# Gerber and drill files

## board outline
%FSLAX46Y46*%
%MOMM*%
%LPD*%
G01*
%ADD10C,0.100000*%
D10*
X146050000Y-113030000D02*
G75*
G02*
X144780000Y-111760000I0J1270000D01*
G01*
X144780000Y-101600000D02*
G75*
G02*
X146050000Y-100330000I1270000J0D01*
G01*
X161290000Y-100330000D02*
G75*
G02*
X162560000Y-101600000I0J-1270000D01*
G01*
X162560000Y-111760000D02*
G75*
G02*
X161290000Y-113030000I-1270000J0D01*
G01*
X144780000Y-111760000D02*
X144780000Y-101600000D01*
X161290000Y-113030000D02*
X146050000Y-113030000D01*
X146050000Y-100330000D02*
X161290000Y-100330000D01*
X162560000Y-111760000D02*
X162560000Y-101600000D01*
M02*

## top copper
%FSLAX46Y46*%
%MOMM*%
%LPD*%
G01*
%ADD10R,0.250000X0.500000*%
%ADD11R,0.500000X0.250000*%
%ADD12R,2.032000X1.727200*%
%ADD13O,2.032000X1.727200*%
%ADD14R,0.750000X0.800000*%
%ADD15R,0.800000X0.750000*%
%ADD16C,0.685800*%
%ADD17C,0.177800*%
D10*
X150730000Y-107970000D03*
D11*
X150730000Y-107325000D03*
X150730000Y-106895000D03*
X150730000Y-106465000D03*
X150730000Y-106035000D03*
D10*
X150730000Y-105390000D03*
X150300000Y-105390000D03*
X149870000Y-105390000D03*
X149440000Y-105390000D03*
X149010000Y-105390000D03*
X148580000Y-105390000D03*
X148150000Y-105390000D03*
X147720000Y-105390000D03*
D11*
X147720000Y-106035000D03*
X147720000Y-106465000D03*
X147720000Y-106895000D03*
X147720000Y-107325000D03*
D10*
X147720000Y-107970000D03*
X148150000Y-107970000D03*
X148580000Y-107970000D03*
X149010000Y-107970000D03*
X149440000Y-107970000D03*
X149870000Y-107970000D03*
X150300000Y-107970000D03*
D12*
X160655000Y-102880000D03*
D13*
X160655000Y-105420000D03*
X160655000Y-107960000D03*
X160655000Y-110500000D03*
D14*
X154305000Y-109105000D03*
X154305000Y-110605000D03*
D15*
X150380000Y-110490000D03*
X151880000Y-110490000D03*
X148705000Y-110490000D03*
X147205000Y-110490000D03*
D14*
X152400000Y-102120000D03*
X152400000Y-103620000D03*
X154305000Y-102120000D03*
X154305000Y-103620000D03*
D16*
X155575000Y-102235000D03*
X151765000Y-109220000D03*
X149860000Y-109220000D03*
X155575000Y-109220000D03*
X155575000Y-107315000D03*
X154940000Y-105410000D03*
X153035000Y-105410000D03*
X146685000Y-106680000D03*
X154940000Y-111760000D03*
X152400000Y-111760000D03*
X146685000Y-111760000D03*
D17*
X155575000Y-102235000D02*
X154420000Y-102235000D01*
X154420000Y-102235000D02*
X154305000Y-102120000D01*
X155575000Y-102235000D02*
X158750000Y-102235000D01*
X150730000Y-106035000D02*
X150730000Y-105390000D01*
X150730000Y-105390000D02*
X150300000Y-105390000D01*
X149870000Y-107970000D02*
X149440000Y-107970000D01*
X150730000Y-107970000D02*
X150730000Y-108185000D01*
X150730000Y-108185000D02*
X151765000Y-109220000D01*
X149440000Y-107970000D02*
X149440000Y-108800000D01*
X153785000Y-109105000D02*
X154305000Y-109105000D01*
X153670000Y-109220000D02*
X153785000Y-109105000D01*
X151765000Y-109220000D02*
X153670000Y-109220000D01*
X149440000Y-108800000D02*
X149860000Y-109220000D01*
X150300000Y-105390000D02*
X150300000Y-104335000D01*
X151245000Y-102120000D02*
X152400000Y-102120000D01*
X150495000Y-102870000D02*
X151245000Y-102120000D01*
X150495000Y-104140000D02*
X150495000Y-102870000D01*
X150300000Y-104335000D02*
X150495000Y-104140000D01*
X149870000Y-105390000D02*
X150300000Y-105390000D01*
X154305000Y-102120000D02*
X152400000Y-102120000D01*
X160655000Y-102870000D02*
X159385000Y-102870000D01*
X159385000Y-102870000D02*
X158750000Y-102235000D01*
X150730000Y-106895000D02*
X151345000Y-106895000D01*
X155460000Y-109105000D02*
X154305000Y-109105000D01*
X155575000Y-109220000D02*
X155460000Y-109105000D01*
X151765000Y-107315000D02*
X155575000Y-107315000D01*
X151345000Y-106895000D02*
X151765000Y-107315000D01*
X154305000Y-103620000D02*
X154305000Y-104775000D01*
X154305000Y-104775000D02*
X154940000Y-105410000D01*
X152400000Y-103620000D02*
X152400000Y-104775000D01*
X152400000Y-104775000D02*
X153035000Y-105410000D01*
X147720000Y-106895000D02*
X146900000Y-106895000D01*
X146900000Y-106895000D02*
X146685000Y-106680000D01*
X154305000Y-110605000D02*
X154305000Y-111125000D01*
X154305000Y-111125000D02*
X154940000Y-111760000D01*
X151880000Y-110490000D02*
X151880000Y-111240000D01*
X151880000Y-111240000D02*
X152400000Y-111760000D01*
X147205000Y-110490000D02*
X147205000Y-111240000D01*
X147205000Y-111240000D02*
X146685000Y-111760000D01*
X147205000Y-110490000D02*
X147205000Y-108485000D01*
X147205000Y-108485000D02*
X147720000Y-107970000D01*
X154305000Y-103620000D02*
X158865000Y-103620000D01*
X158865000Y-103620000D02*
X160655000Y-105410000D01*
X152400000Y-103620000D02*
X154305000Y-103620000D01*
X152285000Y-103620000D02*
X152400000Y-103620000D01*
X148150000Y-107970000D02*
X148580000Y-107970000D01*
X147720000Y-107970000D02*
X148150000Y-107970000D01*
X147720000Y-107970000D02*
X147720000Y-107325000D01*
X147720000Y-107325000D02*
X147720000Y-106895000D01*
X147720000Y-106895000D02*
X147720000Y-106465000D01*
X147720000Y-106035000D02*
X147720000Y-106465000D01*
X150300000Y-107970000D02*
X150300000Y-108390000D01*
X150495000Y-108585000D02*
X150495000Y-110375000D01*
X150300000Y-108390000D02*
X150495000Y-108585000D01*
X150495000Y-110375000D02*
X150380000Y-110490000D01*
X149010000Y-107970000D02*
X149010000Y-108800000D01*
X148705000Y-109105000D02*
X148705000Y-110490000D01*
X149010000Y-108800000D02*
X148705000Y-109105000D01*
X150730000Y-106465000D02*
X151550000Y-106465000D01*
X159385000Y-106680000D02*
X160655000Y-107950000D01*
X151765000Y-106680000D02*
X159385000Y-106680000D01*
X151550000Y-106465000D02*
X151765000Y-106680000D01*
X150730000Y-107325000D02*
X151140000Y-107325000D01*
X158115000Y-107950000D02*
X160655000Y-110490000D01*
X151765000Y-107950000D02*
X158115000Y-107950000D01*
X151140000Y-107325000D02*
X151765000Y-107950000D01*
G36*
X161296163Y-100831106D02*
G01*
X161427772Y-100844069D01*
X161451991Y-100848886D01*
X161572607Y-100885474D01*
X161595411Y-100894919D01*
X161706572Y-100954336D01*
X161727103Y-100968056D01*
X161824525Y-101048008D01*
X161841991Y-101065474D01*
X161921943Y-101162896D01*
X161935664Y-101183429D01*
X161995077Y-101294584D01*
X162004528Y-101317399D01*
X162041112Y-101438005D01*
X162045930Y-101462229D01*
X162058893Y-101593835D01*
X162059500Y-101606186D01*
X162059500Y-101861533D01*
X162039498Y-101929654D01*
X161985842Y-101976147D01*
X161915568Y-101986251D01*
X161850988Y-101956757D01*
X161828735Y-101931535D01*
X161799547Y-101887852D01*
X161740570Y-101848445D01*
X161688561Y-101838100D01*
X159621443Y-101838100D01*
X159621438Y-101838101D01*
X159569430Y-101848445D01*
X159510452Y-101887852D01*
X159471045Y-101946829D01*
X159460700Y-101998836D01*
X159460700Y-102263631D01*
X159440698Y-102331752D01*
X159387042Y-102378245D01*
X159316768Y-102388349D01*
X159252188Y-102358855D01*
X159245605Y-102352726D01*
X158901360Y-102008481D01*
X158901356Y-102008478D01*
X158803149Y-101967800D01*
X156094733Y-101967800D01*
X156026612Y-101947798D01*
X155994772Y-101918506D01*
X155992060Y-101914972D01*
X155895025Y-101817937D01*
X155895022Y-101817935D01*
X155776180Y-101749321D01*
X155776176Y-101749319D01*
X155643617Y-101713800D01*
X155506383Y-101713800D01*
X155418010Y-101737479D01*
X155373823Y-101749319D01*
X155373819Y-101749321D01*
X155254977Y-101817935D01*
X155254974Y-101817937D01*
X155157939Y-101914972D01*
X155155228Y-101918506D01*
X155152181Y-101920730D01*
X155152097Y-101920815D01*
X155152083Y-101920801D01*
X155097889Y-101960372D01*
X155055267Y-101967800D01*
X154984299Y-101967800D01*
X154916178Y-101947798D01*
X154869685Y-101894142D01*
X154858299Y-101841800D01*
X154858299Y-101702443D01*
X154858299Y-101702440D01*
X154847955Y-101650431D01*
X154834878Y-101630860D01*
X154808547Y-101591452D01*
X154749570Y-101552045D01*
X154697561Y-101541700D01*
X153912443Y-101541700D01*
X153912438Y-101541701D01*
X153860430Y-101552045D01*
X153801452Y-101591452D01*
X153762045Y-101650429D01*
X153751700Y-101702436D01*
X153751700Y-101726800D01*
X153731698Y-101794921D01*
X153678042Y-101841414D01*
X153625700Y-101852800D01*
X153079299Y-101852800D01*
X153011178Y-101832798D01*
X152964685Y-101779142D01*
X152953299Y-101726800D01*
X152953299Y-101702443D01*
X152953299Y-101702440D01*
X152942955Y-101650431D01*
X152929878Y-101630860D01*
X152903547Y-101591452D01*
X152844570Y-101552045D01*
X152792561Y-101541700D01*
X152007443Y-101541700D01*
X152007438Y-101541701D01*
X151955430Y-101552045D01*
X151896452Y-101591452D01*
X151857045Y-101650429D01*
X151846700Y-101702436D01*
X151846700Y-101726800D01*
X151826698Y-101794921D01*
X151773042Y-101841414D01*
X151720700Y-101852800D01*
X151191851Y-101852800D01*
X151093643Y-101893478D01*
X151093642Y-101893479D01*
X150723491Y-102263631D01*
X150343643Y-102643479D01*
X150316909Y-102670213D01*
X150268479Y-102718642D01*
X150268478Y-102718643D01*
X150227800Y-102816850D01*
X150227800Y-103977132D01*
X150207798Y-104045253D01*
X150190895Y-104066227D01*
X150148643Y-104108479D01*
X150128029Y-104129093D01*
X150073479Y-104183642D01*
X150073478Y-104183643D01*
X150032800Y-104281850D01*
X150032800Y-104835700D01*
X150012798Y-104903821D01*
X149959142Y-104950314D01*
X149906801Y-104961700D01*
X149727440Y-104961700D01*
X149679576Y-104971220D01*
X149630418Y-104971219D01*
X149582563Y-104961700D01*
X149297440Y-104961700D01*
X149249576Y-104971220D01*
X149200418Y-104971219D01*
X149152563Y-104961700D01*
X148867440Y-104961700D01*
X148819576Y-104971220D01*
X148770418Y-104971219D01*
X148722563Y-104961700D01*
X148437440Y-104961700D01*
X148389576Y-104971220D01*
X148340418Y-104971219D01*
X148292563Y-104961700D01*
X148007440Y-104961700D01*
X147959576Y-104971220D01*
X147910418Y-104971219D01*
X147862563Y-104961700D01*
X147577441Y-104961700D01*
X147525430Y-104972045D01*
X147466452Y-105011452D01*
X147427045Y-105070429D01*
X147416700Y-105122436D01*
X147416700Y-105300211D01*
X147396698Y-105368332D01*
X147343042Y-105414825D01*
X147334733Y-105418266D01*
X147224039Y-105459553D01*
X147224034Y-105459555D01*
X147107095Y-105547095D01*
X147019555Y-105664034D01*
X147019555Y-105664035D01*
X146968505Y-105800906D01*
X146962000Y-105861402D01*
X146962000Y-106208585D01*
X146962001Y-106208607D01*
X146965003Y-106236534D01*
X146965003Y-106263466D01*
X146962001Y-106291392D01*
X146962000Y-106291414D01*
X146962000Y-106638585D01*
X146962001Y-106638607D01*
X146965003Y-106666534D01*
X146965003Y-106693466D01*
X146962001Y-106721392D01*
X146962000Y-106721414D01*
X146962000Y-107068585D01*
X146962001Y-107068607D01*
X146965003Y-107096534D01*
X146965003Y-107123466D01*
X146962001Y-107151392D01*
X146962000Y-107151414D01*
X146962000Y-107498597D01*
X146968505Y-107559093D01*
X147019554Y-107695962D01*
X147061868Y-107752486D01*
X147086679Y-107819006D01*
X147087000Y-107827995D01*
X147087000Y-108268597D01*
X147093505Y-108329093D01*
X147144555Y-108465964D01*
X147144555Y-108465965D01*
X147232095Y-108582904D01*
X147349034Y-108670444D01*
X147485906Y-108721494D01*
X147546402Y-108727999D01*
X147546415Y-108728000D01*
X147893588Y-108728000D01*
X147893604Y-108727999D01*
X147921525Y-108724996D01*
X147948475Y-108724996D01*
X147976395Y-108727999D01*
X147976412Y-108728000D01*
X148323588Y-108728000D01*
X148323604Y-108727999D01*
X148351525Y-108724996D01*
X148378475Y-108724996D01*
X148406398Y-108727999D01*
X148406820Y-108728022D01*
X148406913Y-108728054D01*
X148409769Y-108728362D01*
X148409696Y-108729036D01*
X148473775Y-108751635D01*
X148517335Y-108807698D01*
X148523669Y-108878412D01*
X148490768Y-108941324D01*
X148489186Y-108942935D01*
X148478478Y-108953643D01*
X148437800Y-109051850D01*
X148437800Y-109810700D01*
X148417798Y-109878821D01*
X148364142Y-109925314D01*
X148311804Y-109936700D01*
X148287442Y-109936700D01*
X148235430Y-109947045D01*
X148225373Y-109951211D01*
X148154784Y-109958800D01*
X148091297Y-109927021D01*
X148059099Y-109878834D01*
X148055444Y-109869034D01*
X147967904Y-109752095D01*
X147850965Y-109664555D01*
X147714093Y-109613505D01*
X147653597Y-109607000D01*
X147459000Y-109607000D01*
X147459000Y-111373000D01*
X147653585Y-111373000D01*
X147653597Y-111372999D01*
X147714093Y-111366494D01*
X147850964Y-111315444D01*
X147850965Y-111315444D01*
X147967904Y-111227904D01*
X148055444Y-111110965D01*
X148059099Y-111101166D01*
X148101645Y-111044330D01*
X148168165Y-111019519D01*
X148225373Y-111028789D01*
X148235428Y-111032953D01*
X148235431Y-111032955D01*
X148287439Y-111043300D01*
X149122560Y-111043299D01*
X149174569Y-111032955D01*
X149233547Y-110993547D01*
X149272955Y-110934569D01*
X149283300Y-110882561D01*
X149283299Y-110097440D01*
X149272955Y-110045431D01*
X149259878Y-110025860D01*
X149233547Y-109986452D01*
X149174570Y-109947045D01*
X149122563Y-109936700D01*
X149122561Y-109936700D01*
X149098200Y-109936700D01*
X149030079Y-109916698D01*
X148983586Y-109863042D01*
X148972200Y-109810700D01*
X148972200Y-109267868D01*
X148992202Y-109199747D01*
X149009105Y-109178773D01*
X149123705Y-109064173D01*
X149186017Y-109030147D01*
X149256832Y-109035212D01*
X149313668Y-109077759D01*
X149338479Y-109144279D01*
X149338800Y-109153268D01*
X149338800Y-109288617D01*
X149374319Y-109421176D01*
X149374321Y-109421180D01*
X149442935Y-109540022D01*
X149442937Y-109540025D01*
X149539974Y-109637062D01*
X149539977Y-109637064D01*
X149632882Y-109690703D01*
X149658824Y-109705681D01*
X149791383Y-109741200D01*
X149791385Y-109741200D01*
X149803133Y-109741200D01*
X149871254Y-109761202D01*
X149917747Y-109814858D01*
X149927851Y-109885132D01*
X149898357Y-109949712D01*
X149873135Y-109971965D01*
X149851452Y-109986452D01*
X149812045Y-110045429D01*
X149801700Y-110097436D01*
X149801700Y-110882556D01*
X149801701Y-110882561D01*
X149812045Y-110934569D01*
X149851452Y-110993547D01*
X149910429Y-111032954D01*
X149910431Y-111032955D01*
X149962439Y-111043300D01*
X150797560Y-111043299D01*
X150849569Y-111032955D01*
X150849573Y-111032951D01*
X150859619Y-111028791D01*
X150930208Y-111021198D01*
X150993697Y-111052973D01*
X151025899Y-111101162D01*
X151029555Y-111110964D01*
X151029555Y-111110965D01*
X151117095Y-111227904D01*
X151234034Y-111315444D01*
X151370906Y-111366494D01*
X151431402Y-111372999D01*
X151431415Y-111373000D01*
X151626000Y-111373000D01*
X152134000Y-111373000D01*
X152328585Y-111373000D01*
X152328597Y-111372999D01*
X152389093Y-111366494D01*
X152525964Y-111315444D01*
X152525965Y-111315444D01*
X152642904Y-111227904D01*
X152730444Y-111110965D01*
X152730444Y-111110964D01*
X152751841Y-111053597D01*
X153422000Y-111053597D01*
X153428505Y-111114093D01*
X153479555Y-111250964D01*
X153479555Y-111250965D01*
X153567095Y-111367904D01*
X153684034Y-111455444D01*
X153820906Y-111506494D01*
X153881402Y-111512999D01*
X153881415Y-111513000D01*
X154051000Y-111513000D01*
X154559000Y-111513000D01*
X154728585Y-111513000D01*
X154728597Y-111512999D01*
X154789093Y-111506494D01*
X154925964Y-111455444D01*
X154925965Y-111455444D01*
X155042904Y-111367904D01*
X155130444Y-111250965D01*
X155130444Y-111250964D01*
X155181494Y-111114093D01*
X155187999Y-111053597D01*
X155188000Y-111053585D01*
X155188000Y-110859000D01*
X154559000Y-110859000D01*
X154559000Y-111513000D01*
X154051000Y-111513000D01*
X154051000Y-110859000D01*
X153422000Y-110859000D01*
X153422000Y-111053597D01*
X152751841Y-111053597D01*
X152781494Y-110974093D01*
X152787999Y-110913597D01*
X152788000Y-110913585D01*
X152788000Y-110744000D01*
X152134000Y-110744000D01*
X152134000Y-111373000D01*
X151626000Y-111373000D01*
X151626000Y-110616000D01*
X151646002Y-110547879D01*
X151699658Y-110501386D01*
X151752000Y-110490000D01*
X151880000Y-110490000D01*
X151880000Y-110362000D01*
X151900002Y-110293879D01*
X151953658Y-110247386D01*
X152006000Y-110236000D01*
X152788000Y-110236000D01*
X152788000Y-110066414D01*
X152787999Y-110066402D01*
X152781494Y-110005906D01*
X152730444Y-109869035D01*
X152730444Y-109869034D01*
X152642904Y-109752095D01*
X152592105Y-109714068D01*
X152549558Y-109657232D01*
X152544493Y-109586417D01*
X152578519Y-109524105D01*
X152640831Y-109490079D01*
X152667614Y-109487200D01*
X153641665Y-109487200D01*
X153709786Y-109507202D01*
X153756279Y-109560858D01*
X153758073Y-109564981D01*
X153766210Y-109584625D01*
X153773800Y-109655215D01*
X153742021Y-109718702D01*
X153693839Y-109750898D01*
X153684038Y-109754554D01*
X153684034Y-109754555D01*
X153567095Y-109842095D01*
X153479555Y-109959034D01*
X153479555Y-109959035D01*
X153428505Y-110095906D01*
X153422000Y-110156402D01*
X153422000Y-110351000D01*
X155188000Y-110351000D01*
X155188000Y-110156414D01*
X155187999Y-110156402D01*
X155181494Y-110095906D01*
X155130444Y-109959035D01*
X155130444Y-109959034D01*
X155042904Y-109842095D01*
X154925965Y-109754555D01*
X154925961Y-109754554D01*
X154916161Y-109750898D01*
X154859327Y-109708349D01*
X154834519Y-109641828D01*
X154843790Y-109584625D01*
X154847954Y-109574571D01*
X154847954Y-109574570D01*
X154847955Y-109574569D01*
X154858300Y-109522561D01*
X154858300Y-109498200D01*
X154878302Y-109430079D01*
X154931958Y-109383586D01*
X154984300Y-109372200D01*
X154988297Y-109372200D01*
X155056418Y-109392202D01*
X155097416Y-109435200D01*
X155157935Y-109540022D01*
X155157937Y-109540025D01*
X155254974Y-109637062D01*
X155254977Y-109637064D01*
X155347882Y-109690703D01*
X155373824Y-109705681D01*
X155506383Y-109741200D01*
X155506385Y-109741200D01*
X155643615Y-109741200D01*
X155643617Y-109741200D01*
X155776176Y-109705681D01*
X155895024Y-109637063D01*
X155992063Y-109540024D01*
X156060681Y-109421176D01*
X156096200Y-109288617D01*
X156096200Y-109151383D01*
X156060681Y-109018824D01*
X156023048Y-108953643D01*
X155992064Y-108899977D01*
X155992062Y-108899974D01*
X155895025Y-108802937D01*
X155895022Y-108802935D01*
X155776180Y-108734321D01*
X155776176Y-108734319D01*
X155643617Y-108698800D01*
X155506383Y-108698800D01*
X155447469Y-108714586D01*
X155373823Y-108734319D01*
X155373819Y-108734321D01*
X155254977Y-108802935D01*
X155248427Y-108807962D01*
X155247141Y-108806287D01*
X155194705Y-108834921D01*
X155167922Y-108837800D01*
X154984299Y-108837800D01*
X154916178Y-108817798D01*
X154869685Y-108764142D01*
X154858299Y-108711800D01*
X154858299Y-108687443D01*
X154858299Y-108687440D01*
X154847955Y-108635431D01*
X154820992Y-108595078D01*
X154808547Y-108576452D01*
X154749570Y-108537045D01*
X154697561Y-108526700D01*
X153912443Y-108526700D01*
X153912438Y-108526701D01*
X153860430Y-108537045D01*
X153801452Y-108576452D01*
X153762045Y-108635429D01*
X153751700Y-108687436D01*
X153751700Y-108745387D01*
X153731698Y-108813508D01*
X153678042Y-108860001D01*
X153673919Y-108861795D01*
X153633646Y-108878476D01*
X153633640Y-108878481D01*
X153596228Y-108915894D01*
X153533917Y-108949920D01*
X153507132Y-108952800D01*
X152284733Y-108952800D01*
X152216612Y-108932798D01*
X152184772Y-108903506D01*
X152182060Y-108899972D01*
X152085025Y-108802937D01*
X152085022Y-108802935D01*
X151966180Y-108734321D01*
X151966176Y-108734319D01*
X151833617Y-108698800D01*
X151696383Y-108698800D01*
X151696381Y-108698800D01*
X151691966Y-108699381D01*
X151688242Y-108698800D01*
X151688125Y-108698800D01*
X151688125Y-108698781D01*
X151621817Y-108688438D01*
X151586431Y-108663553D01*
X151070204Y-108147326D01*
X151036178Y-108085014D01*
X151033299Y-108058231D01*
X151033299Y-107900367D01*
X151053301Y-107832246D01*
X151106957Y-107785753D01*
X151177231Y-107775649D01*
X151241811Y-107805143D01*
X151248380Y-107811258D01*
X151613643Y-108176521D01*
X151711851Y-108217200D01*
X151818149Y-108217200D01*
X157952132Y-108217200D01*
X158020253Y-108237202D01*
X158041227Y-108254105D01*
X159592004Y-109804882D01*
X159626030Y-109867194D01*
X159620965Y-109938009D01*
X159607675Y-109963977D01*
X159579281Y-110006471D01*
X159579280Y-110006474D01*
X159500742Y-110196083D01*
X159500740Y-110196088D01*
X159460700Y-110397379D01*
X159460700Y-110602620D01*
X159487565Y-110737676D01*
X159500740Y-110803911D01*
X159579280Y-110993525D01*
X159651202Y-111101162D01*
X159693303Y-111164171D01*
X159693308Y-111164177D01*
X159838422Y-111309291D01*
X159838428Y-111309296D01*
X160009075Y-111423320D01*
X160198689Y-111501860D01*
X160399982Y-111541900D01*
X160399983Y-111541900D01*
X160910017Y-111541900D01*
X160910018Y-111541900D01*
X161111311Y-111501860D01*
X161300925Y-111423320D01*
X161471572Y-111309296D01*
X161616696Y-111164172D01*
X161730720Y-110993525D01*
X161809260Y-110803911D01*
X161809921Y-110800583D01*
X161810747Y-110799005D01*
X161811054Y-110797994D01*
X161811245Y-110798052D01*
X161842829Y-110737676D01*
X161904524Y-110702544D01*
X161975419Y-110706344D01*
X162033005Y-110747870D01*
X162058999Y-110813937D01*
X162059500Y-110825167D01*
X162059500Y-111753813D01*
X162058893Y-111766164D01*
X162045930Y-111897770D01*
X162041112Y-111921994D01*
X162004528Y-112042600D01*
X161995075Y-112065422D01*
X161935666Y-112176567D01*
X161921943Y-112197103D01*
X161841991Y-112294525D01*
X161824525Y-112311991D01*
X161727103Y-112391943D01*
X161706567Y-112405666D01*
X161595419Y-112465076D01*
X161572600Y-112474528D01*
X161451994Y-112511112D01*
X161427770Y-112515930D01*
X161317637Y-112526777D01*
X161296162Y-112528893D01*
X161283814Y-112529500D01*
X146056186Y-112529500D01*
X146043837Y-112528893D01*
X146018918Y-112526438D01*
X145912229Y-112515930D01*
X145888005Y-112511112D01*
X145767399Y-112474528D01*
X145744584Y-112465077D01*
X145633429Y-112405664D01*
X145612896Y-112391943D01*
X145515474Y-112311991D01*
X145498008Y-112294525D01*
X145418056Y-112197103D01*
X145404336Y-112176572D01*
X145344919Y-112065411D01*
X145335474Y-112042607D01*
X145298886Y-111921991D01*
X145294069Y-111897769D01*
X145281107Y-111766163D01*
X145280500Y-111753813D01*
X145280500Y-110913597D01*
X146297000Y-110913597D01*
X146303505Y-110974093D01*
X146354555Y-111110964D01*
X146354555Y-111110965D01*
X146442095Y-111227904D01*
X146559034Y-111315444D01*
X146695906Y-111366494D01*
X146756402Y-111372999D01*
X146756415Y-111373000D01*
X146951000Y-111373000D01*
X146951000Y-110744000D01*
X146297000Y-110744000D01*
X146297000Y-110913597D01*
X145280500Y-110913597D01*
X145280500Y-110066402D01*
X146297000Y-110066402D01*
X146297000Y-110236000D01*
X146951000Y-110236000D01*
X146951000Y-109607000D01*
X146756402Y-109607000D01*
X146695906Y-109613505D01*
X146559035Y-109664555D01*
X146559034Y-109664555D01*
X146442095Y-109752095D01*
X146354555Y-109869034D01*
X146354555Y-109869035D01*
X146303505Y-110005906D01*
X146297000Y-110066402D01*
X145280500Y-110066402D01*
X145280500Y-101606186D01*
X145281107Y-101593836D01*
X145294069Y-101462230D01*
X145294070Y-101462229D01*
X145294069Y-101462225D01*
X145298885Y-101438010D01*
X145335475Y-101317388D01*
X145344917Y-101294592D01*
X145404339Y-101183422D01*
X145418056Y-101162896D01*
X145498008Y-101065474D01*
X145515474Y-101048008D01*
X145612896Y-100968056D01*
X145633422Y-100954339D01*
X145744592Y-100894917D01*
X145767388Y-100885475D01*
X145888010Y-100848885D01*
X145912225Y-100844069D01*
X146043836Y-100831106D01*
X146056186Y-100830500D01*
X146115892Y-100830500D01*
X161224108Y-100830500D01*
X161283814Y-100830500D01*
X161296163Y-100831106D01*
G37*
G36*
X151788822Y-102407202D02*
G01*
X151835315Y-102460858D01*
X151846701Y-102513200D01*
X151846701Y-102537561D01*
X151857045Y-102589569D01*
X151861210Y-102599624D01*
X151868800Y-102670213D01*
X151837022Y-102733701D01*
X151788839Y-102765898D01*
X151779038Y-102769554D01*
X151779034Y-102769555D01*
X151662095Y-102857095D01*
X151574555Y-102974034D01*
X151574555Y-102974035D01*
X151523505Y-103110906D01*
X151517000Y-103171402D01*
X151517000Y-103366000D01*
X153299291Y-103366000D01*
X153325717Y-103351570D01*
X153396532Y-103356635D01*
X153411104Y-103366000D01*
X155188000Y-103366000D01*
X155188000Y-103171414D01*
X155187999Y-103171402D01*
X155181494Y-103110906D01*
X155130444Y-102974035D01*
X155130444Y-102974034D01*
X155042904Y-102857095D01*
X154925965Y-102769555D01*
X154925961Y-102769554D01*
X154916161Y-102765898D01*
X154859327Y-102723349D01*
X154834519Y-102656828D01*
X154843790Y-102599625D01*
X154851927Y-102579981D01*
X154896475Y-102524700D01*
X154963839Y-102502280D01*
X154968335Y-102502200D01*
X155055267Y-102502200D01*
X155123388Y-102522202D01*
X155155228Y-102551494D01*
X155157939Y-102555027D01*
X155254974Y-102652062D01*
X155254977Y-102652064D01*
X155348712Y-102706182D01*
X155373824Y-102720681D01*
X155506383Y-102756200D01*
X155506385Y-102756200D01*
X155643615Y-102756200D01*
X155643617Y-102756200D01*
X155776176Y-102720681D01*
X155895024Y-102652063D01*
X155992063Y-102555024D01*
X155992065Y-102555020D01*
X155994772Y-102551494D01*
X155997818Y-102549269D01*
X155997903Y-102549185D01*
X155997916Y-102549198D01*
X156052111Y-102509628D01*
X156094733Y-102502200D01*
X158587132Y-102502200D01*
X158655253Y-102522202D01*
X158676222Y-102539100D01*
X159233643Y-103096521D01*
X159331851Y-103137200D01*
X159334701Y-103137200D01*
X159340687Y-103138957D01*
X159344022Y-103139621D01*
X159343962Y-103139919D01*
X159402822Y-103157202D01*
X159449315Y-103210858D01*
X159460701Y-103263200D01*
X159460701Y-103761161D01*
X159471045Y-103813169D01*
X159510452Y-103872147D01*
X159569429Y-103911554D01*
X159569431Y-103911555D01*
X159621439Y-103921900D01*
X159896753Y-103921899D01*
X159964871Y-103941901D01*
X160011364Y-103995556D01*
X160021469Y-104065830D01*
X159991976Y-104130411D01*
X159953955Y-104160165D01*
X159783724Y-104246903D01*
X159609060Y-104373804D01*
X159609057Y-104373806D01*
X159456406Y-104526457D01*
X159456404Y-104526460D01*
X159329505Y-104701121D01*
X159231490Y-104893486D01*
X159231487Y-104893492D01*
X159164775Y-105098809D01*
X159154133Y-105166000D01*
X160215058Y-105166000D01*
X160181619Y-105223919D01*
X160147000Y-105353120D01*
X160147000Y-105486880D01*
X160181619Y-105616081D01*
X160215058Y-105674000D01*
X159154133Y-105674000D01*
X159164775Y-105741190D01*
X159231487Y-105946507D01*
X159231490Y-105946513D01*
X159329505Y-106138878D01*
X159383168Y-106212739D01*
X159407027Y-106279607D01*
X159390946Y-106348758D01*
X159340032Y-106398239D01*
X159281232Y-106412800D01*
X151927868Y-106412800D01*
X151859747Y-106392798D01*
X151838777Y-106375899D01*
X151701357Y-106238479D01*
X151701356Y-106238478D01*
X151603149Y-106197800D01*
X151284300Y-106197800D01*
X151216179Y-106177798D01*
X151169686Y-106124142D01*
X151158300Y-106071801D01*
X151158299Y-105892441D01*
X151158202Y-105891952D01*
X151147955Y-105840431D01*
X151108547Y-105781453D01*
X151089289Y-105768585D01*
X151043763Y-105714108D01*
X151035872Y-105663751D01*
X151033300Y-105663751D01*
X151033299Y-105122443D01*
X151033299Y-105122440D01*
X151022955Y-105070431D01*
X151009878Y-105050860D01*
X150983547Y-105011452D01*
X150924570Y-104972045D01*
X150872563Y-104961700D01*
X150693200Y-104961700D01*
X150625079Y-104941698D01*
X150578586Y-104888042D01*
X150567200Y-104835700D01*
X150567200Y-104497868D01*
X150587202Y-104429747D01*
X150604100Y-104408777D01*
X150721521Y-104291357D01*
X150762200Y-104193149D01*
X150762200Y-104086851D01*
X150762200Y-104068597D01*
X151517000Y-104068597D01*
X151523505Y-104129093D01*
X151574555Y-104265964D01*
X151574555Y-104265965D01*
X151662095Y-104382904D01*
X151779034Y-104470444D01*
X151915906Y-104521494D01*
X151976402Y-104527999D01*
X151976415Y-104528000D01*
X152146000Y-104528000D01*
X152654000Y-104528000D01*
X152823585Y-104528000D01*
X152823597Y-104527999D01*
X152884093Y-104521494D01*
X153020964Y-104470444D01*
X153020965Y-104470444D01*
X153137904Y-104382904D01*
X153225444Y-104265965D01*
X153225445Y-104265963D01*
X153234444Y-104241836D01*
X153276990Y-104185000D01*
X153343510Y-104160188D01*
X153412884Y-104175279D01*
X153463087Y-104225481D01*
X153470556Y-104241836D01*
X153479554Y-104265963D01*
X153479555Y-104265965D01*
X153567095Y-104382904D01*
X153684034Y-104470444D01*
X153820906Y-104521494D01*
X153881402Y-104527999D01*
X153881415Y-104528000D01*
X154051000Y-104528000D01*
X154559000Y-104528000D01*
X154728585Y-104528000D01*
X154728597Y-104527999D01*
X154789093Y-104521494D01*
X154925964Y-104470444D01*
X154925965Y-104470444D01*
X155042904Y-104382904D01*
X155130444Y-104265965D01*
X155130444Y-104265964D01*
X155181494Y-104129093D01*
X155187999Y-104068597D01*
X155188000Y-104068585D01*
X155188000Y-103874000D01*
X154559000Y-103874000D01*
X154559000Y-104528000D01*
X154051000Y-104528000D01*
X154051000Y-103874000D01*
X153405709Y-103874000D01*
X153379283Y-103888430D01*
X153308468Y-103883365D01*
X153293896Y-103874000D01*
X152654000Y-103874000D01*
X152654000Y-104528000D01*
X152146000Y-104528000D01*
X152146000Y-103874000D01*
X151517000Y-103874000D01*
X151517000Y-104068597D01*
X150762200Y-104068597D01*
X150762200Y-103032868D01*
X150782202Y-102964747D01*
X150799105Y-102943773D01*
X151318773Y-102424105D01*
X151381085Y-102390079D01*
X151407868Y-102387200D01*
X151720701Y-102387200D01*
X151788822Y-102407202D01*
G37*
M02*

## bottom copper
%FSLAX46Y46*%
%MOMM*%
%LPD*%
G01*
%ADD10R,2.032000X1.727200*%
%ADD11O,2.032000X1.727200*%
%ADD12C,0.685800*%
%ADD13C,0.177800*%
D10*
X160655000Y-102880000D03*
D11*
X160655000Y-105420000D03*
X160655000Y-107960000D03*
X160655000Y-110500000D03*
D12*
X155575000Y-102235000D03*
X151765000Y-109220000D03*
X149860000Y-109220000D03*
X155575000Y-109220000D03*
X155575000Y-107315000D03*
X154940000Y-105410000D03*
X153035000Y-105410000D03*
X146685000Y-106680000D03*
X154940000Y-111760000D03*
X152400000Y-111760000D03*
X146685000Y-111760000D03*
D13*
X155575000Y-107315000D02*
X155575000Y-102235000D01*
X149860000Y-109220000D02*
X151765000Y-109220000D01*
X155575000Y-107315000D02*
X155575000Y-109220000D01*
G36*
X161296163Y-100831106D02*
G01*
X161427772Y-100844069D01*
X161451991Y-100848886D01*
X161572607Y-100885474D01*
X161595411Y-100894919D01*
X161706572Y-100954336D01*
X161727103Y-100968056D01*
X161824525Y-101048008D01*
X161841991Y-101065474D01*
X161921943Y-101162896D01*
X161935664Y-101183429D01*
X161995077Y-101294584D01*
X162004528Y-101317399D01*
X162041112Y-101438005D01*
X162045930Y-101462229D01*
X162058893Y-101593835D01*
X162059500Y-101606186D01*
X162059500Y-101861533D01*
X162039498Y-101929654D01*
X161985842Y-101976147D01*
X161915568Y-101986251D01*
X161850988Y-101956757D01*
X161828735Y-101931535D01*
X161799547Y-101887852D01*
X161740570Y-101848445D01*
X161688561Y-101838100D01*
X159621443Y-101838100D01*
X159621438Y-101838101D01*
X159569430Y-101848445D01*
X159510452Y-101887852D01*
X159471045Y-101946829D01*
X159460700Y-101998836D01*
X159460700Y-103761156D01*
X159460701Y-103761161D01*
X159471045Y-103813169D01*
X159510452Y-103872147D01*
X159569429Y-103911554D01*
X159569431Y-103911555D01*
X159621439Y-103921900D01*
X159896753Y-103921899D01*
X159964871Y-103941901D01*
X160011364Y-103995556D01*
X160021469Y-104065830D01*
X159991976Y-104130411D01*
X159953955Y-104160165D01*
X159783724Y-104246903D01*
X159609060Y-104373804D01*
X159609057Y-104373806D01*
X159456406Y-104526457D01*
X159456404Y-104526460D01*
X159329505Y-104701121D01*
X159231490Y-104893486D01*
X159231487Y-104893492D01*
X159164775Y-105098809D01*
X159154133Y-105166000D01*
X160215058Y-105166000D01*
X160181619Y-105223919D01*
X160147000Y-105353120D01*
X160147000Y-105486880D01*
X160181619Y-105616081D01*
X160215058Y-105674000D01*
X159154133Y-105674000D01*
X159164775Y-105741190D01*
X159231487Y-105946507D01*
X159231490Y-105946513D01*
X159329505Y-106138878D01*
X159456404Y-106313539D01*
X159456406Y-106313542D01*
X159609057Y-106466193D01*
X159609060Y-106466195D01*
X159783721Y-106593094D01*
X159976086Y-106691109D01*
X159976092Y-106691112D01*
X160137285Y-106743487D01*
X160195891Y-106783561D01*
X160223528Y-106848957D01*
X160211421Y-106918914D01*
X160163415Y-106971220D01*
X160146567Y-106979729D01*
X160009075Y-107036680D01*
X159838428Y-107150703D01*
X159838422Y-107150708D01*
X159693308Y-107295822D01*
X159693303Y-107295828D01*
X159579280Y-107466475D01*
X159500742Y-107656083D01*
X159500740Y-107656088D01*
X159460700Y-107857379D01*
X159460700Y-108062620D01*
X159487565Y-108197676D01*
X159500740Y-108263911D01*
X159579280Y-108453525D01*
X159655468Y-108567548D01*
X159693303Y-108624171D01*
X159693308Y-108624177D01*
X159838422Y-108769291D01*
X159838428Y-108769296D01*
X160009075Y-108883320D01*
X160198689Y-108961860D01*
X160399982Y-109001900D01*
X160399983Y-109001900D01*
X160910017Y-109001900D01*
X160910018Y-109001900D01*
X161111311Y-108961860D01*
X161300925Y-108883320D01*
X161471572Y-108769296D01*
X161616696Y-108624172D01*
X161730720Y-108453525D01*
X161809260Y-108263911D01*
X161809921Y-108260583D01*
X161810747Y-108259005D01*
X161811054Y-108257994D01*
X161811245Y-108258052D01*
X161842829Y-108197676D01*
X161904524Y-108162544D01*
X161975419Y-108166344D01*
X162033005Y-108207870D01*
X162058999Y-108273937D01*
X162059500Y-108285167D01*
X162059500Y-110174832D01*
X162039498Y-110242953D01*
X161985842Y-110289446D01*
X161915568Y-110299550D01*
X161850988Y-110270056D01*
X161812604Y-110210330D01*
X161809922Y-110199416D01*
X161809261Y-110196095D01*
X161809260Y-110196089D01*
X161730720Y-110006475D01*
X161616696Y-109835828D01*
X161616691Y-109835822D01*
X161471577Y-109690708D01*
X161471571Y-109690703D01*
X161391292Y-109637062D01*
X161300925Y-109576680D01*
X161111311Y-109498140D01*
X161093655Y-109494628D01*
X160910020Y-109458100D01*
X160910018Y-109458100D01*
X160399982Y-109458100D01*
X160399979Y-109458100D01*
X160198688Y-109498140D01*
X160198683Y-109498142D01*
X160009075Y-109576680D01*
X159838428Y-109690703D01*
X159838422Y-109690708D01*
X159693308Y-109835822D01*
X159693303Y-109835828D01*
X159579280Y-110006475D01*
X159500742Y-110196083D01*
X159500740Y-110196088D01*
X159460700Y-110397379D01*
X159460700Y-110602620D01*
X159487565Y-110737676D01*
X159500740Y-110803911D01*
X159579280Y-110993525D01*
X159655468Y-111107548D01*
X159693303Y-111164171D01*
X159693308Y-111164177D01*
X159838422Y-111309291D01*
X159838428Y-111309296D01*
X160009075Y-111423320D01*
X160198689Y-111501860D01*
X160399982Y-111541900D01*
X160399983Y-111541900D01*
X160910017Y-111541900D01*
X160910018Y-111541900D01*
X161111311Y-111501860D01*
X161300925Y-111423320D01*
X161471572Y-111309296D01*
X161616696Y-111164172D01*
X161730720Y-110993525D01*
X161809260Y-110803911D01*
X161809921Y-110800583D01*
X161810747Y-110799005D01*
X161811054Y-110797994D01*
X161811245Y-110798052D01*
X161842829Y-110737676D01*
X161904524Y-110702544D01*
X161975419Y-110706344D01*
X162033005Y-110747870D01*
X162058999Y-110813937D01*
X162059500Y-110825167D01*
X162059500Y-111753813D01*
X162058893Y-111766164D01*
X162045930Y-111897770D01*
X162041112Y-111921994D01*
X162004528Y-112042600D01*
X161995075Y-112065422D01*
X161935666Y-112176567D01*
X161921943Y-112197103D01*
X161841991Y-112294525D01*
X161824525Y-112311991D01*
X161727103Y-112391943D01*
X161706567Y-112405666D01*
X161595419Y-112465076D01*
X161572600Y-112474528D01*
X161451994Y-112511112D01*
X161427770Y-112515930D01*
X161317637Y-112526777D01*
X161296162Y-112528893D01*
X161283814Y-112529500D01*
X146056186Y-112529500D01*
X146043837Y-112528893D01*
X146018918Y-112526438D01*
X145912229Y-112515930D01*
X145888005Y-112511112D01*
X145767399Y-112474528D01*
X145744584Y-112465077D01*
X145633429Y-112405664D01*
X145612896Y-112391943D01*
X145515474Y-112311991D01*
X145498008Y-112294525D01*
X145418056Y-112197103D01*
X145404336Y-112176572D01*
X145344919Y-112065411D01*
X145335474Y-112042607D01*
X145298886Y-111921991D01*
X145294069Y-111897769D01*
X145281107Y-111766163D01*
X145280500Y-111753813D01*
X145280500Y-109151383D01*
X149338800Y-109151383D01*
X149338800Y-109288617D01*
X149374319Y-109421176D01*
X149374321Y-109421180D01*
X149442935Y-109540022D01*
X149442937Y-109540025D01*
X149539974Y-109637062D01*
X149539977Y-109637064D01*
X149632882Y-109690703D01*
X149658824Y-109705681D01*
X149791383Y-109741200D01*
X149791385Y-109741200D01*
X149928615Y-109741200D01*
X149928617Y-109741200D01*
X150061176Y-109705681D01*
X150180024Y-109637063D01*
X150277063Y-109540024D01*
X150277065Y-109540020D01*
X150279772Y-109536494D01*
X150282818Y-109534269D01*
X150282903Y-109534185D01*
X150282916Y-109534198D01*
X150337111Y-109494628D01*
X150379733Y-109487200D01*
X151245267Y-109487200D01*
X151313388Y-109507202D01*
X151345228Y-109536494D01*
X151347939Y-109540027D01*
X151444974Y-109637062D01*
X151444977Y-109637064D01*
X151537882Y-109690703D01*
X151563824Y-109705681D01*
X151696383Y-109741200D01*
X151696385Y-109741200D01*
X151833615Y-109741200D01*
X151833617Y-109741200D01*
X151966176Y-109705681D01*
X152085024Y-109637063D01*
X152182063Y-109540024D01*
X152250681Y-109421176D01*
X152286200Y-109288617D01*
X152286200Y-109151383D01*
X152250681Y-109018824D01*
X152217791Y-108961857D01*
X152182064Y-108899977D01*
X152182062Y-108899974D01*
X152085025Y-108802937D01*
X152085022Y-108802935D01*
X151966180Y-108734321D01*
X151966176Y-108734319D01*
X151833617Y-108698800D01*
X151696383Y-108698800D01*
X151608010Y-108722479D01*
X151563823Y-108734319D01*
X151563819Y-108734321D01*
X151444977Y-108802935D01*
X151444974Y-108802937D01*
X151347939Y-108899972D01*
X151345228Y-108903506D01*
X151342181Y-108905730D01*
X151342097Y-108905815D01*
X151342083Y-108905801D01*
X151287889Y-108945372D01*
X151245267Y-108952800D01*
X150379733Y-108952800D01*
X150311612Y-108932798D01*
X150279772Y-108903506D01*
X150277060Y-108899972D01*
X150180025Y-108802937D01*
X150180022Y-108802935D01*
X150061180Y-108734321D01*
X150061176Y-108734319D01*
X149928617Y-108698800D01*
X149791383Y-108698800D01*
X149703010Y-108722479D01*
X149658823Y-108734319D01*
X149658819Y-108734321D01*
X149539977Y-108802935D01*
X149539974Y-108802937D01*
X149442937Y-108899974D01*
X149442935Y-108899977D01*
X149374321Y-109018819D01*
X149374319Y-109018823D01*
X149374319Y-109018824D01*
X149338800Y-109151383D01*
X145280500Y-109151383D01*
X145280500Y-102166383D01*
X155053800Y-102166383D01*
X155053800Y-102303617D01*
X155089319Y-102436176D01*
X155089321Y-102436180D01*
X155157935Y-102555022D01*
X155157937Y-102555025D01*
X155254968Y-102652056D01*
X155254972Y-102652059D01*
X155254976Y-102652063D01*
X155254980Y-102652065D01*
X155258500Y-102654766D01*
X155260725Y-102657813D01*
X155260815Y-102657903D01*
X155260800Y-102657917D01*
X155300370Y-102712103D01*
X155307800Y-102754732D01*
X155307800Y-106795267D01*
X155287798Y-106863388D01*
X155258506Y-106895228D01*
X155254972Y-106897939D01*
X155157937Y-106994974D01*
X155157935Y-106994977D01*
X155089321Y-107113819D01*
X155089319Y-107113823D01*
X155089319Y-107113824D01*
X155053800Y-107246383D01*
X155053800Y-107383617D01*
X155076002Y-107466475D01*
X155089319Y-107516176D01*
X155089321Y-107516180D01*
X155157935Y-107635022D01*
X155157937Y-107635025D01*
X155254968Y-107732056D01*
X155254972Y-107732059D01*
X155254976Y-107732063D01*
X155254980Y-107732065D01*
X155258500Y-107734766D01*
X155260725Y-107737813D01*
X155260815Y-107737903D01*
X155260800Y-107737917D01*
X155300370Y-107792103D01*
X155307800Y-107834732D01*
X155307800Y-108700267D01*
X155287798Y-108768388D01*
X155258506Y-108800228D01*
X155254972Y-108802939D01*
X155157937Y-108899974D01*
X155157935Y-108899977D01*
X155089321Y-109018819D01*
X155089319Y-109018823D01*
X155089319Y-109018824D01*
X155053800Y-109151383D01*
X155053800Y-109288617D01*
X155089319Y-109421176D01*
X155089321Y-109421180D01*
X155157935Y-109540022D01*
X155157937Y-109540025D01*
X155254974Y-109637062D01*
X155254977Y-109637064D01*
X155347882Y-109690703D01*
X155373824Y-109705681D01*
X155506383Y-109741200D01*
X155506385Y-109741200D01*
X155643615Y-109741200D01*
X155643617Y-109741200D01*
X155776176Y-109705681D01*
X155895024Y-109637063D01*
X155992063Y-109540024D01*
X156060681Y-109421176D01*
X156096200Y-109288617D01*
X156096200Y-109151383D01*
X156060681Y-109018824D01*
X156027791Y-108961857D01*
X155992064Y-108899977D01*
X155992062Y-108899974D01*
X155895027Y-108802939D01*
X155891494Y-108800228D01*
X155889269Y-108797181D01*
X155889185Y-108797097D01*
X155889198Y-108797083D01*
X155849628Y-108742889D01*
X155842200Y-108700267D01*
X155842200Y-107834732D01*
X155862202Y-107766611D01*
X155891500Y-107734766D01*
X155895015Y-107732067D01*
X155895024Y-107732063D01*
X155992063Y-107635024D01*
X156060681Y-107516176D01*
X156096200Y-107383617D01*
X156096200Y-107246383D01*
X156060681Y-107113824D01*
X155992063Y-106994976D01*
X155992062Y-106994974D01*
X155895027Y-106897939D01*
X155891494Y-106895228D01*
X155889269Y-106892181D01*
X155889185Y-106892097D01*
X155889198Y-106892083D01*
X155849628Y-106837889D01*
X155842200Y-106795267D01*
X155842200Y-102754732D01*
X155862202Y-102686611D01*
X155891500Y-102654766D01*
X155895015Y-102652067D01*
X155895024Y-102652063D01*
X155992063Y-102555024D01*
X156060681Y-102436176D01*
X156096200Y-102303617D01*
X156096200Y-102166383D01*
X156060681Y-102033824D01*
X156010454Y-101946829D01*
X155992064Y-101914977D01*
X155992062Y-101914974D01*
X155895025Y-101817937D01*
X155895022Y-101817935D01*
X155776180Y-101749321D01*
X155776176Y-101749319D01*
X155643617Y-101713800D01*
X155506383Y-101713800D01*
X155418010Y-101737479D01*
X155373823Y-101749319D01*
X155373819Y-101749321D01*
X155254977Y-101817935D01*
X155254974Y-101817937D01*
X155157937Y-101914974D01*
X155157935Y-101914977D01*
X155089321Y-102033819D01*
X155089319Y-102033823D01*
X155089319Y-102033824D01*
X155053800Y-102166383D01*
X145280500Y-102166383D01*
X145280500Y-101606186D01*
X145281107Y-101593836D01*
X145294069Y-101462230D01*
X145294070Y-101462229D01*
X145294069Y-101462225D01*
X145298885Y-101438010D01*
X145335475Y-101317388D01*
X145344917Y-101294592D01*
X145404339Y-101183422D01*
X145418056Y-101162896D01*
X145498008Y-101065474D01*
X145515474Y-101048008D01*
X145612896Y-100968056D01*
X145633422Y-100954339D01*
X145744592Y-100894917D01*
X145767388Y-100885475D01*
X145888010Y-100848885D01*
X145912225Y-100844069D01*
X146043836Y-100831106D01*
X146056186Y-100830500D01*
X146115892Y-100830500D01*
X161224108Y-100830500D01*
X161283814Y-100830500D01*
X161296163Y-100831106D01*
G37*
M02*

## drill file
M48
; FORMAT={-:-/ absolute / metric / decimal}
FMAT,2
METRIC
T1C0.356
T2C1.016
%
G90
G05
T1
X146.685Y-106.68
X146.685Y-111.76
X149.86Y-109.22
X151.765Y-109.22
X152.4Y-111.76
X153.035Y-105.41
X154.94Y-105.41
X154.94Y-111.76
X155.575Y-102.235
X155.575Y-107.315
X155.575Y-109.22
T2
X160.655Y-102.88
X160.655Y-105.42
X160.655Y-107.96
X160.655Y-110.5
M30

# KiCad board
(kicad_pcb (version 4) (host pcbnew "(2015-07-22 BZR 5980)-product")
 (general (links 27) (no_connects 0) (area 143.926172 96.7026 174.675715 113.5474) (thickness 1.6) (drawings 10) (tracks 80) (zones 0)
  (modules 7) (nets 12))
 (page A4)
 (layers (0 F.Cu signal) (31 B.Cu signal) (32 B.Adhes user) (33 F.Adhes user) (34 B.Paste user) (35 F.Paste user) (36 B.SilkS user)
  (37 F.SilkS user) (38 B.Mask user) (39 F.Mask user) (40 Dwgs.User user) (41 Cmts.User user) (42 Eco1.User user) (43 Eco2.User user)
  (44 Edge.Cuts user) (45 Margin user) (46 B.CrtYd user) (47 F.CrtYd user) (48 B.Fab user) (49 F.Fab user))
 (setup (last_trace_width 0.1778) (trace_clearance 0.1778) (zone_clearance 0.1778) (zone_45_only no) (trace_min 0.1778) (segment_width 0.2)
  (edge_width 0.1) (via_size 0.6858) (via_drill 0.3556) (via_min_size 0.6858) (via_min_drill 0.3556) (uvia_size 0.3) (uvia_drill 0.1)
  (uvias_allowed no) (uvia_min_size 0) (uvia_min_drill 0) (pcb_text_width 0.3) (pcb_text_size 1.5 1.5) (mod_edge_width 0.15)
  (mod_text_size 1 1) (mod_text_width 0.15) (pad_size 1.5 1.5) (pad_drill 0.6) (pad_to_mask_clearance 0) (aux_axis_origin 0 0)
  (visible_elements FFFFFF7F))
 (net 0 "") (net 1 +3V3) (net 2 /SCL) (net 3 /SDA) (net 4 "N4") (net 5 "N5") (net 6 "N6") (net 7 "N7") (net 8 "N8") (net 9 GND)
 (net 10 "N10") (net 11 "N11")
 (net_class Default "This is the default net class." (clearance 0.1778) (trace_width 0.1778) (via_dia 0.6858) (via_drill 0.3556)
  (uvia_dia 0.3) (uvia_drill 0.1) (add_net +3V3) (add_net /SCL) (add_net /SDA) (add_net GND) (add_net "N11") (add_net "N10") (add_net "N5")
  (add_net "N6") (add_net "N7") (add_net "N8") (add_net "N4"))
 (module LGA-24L (layer F.Cu) (at 149.225 106.68 180)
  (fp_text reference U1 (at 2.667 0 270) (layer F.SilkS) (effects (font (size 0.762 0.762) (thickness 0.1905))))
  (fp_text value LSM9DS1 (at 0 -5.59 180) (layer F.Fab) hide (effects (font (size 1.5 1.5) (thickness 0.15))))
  (pad 1 smd rect (at -1.505 -1.29 180) (size 0.25 0.5) (layers F.Cu F.Paste F.Mask) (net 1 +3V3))
  (pad 2 smd rect (at -1.505 -0.645 180) (size 0.5 0.25) (layers F.Cu F.Paste F.Mask) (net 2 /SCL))
  (pad 3 smd rect (at -1.505 -0.215 180) (size 0.5 0.25) (layers F.Cu F.Paste F.Mask) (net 1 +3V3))
  (pad 4 smd rect (at -1.505 0.215 180) (size 0.5 0.25) (layers F.Cu F.Paste F.Mask) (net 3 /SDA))
  (pad 5 smd rect (at -1.505 0.645 180) (size 0.5 0.25) (layers F.Cu F.Paste F.Mask) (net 1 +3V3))
  (pad 6 smd rect (at -1.505 1.29 180) (size 0.25 0.5) (layers F.Cu F.Paste F.Mask) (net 1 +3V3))
  (pad 7 smd rect (at -1.075 1.29 180) (size 0.25 0.5) (layers F.Cu F.Paste F.Mask) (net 1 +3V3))
  (pad 8 smd rect (at -0.645 1.29 180) (size 0.25 0.5) (layers F.Cu F.Paste F.Mask) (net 1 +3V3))
  (pad 9 smd rect (at -0.215 1.29 180) (size 0.25 0.5) (layers F.Cu F.Paste F.Mask) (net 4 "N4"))
  (pad 10 smd rect (at 0.215 1.29 180) (size 0.25 0.5) (layers F.Cu F.Paste F.Mask) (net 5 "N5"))
  (pad 11 smd rect (at 0.645 1.29 180) (size 0.25 0.5) (layers F.Cu F.Paste F.Mask) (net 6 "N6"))
  (pad 12 smd rect (at 1.075 1.29 180) (size 0.25 0.5) (layers F.Cu F.Paste F.Mask) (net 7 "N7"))
  (pad 13 smd rect (at 1.505 1.29 180) (size 0.25 0.5) (layers F.Cu F.Paste F.Mask) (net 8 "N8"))
  (pad 14 smd rect (at 1.505 0.645 180) (size 0.5 0.25) (layers F.Cu F.Paste F.Mask) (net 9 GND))
  (pad 15 smd rect (at 1.505 0.215 180) (size 0.5 0.25) (layers F.Cu F.Paste F.Mask) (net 9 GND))
  (pad 16 smd rect (at 1.505 -0.215 180) (size 0.5 0.25) (layers F.Cu F.Paste F.Mask) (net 9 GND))
  (pad 17 smd rect (at 1.505 -0.645 180) (size 0.5 0.25) (layers F.Cu F.Paste F.Mask) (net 9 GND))
  (pad 18 smd rect (at 1.505 -1.29 180) (size 0.25 0.5) (layers F.Cu F.Paste F.Mask) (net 9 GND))
  (pad 19 smd rect (at 1.075 -1.29 180) (size 0.25 0.5) (layers F.Cu F.Paste F.Mask) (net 9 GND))
  (pad 20 smd rect (at 0.645 -1.29 180) (size 0.25 0.5) (layers F.Cu F.Paste F.Mask) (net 9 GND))
  (pad 21 smd rect (at 0.215 -1.29 180) (size 0.25 0.5) (layers F.Cu F.Paste F.Mask) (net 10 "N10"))
  (pad 22 smd rect (at -0.215 -1.29 180) (size 0.25 0.5) (layers F.Cu F.Paste F.Mask) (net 1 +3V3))
  (pad 23 smd rect (at -0.645 -1.29 180) (size 0.25 0.5) (layers F.Cu F.Paste F.Mask) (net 1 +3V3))
  (pad 24 smd rect (at -1.075 -1.29 180) (size 0.25 0.5) (layers F.Cu F.Paste F.Mask) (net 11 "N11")))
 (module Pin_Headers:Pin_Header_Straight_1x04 (layer F.Cu) (at 160.655 106.68)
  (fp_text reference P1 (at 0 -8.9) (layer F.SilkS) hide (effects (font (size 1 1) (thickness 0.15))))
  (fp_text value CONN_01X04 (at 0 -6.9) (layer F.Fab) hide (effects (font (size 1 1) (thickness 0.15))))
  (pad 1 thru_hole rect (at 0 -3.8) (size 2.032 1.7272) (drill 1.016) (layers *.Cu *.Mask F.SilkS) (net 1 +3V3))
  (pad 2 thru_hole oval (at 0 -1.26) (size 2.032 1.7272) (drill 1.016) (layers *.Cu *.Mask F.SilkS) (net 9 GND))
  (pad 3 thru_hole oval (at 0 1.28) (size 2.032 1.7272) (drill 1.016) (layers *.Cu *.Mask F.SilkS) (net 3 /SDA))
  (pad 4 thru_hole oval (at 0 3.82) (size 2.032 1.7272) (drill 1.016) (layers *.Cu *.Mask F.SilkS) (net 2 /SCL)))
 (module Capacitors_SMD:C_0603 (layer F.Cu) (at 154.305 109.855 270)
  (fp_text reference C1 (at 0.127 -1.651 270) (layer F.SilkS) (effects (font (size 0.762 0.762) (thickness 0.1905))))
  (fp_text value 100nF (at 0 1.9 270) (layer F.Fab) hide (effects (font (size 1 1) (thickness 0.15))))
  (pad 1 smd rect (at -0.75 0 270) (size 0.8 0.75) (layers F.Cu F.Paste F.Mask) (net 1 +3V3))
  (pad 2 smd rect (at 0.75 0 270) (size 0.8 0.75) (layers F.Cu F.Paste F.Mask) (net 9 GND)))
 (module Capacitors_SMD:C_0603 (layer F.Cu) (at 151.13 110.49)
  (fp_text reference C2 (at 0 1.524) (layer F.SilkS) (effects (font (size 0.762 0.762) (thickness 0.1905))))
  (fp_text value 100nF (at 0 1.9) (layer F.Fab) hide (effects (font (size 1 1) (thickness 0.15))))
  (pad 1 smd rect (at -0.75 0) (size 0.8 0.75) (layers F.Cu F.Paste F.Mask) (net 11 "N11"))
  (pad 2 smd rect (at 0.75 0) (size 0.8 0.75) (layers F.Cu F.Paste F.Mask) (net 9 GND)))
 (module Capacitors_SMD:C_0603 (layer F.Cu) (at 147.955 110.49 180)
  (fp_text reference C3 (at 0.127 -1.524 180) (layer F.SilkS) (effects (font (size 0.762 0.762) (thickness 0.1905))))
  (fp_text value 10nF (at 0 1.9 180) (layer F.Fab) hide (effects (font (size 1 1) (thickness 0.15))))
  (pad 1 smd rect (at -0.75 0 180) (size 0.8 0.75) (layers F.Cu F.Paste F.Mask) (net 10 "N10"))
  (pad 2 smd rect (at 0.75 0 180) (size 0.8 0.75) (layers F.Cu F.Paste F.Mask) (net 9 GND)))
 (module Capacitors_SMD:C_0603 (layer F.Cu) (at 152.4 102.87 270)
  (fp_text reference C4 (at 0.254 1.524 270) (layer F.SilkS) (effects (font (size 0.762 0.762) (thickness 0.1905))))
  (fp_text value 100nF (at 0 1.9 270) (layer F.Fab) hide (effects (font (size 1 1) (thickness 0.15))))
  (pad 1 smd rect (at -0.75 0 270) (size 0.8 0.75) (layers F.Cu F.Paste F.Mask) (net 1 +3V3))
  (pad 2 smd rect (at 0.75 0 270) (size 0.8 0.75) (layers F.Cu F.Paste F.Mask) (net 9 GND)))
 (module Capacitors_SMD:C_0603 (layer F.Cu) (at 154.305 102.87 270)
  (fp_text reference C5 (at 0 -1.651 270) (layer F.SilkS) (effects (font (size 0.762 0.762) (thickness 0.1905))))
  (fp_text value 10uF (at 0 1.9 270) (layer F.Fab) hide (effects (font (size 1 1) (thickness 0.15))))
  (pad 1 smd rect (at -0.75 0 270) (size 0.8 0.75) (layers F.Cu F.Paste F.Mask) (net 1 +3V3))
  (pad 2 smd rect (at 0.75 0 270) (size 0.8 0.75) (layers F.Cu F.Paste F.Mask) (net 9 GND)))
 (gr_arc (start 146.05 111.76) (end 146.05 113.03) (angle 90) (layer Edge.Cuts) (width 0.1))
 (gr_arc (start 146.05 101.6) (end 144.78 101.6) (angle 90) (layer Edge.Cuts) (width 0.1))
 (gr_arc (start 161.29 101.6) (end 161.29 100.33) (angle 90) (layer Edge.Cuts) (width 0.1))
 (gr_arc (start 161.29 111.76) (end 162.56 111.76) (angle 90) (layer Edge.Cuts) (width 0.1))
 (gr_line (start 144.78 111.76) (end 144.78 101.6) (angle 90) (layer Edge.Cuts) (width 0.1))
 (gr_line (start 161.29 113.03) (end 146.05 113.03) (angle 90) (layer Edge.Cuts) (width 0.1))
 (gr_line (start 146.05 100.33) (end 161.29 100.33) (angle 90) (layer Edge.Cuts) (width 0.1))
 (gr_line (start 162.56 111.76) (end 162.56 101.6) (angle 90) (layer Edge.Cuts) (width 0.1))
 (segment (start 155.575 102.235) (end 154.42 102.235) (width 0.1778) (layer F.Cu) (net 1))
 (segment (start 154.42 102.235) (end 154.305 102.12) (width 0.1778) (layer F.Cu) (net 1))
 (segment (start 155.575 107.315) (end 155.575 102.235) (width 0.1778) (layer B.Cu) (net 1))
 (segment (start 155.575 102.235) (end 158.75 102.235) (width 0.1778) (layer F.Cu) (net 1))
 (via (at 155.575 102.235) (size 0.6858) (drill 0.3556) (layers F.Cu B.Cu) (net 1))
 (segment (start 150.73 106.035) (end 150.73 105.39) (width 0.1778) (layer F.Cu) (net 1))
 (segment (start 150.73 105.39) (end 150.3 105.39) (width 0.1778) (layer F.Cu) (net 1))
 (segment (start 149.87 107.97) (end 149.44 107.97) (width 0.1778) (layer F.Cu) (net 1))
 (segment (start 150.73 107.97) (end 150.73 108.185) (width 0.1778) (layer F.Cu) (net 1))
 (segment (start 150.73 108.185) (end 151.765 109.22) (width 0.1778) (layer F.Cu) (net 1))
 (segment (start 149.44 107.97) (end 149.44 108.8) (width 0.1778) (layer F.Cu) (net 1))
 (segment (start 153.785 109.105) (end 154.305 109.105) (width 0.1778) (layer F.Cu) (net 1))
 (segment (start 153.67 109.22) (end 153.785 109.105) (width 0.1778) (layer F.Cu) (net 1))
 (segment (start 151.765 109.22) (end 153.67 109.22) (width 0.1778) (layer F.Cu) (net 1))
 (via (at 151.765 109.22) (size 0.6858) (drill 0.3556) (layers F.Cu B.Cu) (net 1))
 (segment (start 149.86 109.22) (end 151.765 109.22) (width 0.1778) (layer B.Cu) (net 1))
 (via (at 149.86 109.22) (size 0.6858) (drill 0.3556) (layers F.Cu B.Cu) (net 1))
 (segment (start 149.44 108.8) (end 149.86 109.22) (width 0.1778) (layer F.Cu) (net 1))
 (segment (start 150.3 105.39) (end 150.3 104.335) (width 0.1778) (layer F.Cu) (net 1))
 (segment (start 151.245 102.12) (end 152.4 102.12) (width 0.1778) (layer F.Cu) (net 1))
 (segment (start 150.495 102.87) (end 151.245 102.12) (width 0.1778) (layer F.Cu) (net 1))
 (segment (start 150.495 104.14) (end 150.495 102.87) (width 0.1778) (layer F.Cu) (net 1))
 (segment (start 150.3 104.335) (end 150.495 104.14) (width 0.1778) (layer F.Cu) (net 1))
 (segment (start 149.87 105.39) (end 150.3 105.39) (width 0.1778) (layer F.Cu) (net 1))
 (segment (start 154.305 102.12) (end 152.4 102.12) (width 0.1778) (layer F.Cu) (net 1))
 (segment (start 160.655 102.87) (end 159.385 102.87) (width 0.1778) (layer F.Cu) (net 1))
 (segment (start 159.385 102.87) (end 158.75 102.235) (width 0.1778) (layer F.Cu) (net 1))
 (segment (start 150.73 106.895) (end 151.345 106.895) (width 0.1778) (layer F.Cu) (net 1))
 (segment (start 155.46 109.105) (end 154.305 109.105) (width 0.1778) (layer F.Cu) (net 1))
 (segment (start 155.575 109.22) (end 155.46 109.105) (width 0.1778) (layer F.Cu) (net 1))
 (via (at 155.575 109.22) (size 0.6858) (drill 0.3556) (layers F.Cu B.Cu) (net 1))
 (segment (start 155.575 107.315) (end 155.575 109.22) (width 0.1778) (layer B.Cu) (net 1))
 (via (at 155.575 107.315) (size 0.6858) (drill 0.3556) (layers F.Cu B.Cu) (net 1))
 (segment (start 151.765 107.315) (end 155.575 107.315) (width 0.1778) (layer F.Cu) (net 1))
 (segment (start 151.345 106.895) (end 151.765 107.315) (width 0.1778) (layer F.Cu) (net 1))
 (segment (start 154.305 103.62) (end 154.305 104.775) (width 0.1778) (layer F.Cu) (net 9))
 (via (at 154.94 105.41) (size 0.6858) (drill 0.3556) (layers F.Cu B.Cu) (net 9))
 (segment (start 154.305 104.775) (end 154.94 105.41) (width 0.1778) (layer F.Cu) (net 9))
 (segment (start 152.4 103.62) (end 152.4 104.775) (width 0.1778) (layer F.Cu) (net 9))
 (via (at 153.035 105.41) (size 0.6858) (drill 0.3556) (layers F.Cu B.Cu) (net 9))
 (segment (start 152.4 104.775) (end 153.035 105.41) (width 0.1778) (layer F.Cu) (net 9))
 (segment (start 147.72 106.895) (end 146.9 106.895) (width 0.1778) (layer F.Cu) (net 9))
 (via (at 146.685 106.68) (size 0.6858) (drill 0.3556) (layers F.Cu B.Cu) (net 9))
 (segment (start 146.9 106.895) (end 146.685 106.68) (width 0.1778) (layer F.Cu) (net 9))
 (segment (start 154.305 110.605) (end 154.305 111.125) (width 0.1778) (layer F.Cu) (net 9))
 (via (at 154.94 111.76) (size 0.6858) (drill 0.3556) (layers F.Cu B.Cu) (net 9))
 (segment (start 154.305 111.125) (end 154.94 111.76) (width 0.1778) (layer F.Cu) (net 9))
 (segment (start 151.88 110.49) (end 151.88 111.24) (width 0.1778) (layer F.Cu) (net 9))
 (via (at 152.4 111.76) (size 0.6858) (drill 0.3556) (layers F.Cu B.Cu) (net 9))
 (segment (start 151.88 111.24) (end 152.4 111.76) (width 0.1778) (layer F.Cu) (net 9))
 (segment (start 147.205 110.49) (end 147.205 111.24) (width 0.1778) (layer F.Cu) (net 9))
 (via (at 146.685 111.76) (size 0.6858) (drill 0.3556) (layers F.Cu B.Cu) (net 9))
 (segment (start 147.205 111.24) (end 146.685 111.76) (width 0.1778) (layer F.Cu) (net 9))
 (segment (start 147.205 110.49) (end 147.205 108.485) (width 0.1778) (layer F.Cu) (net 9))
 (segment (start 147.205 108.485) (end 147.72 107.97) (width 0.1778) (layer F.Cu) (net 9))
 (segment (start 154.305 103.62) (end 158.865 103.62) (width 0.1778) (layer F.Cu) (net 9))
 (segment (start 158.865 103.62) (end 160.655 105.41) (width 0.1778) (layer F.Cu) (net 9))
 (segment (start 152.4 103.62) (end 154.305 103.62) (width 0.1778) (layer F.Cu) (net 9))
 (segment (start 152.285 103.62) (end 152.4 103.62) (width 0.1778) (layer F.Cu) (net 9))
 (segment (start 148.15 107.97) (end 148.58 107.97) (width 0.1778) (layer F.Cu) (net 9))
 (segment (start 147.72 107.97) (end 148.15 107.97) (width 0.1778) (layer F.Cu) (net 9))
 (segment (start 147.72 107.97) (end 147.72 107.325) (width 0.1778) (layer F.Cu) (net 9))
 (segment (start 147.72 107.325) (end 147.72 106.895) (width 0.1778) (layer F.Cu) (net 9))
 (segment (start 147.72 106.895) (end 147.72 106.465) (width 0.1778) (layer F.Cu) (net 9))
 (segment (start 147.72 106.035) (end 147.72 106.465) (width 0.1778) (layer F.Cu) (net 9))
 (segment (start 150.3 107.97) (end 150.3 108.39) (width 0.1778) (layer F.Cu) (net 11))
 (segment (start 150.495 108.585) (end 150.495 110.375) (width 0.1778) (layer F.Cu) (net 11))
 (segment (start 150.3 108.39) (end 150.495 108.585) (width 0.1778) (layer F.Cu) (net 11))
 (segment (start 150.495 110.375) (end 150.38 110.49) (width 0.1778) (layer F.Cu) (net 11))
 (segment (start 149.01 107.97) (end 149.01 108.8) (width 0.1778) (layer F.Cu) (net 10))
 (segment (start 148.705 109.105) (end 148.705 110.49) (width 0.1778) (layer F.Cu) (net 10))
 (segment (start 149.01 108.8) (end 148.705 109.105) (width 0.1778) (layer F.Cu) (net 10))
 (segment (start 150.73 106.465) (end 151.55 106.465) (width 0.1778) (layer F.Cu) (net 3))
 (segment (start 159.385 106.68) (end 160.655 107.95) (width 0.1778) (layer F.Cu) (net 3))
 (segment (start 151.765 106.68) (end 159.385 106.68) (width 0.1778) (layer F.Cu) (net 3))
 (segment (start 151.55 106.465) (end 151.765 106.68) (width 0.1778) (layer F.Cu) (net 3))
 (segment (start 150.73 107.325) (end 151.14 107.325) (width 0.1778) (layer F.Cu) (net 2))
 (segment (start 158.115 107.95) (end 160.655 110.49) (width 0.1778) (layer F.Cu) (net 2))
 (segment (start 151.765 107.95) (end 158.115 107.95) (width 0.1778) (layer F.Cu) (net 2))
 (segment (start 151.14 107.325) (end 151.765 107.95) (width 0.1778) (layer F.Cu) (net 2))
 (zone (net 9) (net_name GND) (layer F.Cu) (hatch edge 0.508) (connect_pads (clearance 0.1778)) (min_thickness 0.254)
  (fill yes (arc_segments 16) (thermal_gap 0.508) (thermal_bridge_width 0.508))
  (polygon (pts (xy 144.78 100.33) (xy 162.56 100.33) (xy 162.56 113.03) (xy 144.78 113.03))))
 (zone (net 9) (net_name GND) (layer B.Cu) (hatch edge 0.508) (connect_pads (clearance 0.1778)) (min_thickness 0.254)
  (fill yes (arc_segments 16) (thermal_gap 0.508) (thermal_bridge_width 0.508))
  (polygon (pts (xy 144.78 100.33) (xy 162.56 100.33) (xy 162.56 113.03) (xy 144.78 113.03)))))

